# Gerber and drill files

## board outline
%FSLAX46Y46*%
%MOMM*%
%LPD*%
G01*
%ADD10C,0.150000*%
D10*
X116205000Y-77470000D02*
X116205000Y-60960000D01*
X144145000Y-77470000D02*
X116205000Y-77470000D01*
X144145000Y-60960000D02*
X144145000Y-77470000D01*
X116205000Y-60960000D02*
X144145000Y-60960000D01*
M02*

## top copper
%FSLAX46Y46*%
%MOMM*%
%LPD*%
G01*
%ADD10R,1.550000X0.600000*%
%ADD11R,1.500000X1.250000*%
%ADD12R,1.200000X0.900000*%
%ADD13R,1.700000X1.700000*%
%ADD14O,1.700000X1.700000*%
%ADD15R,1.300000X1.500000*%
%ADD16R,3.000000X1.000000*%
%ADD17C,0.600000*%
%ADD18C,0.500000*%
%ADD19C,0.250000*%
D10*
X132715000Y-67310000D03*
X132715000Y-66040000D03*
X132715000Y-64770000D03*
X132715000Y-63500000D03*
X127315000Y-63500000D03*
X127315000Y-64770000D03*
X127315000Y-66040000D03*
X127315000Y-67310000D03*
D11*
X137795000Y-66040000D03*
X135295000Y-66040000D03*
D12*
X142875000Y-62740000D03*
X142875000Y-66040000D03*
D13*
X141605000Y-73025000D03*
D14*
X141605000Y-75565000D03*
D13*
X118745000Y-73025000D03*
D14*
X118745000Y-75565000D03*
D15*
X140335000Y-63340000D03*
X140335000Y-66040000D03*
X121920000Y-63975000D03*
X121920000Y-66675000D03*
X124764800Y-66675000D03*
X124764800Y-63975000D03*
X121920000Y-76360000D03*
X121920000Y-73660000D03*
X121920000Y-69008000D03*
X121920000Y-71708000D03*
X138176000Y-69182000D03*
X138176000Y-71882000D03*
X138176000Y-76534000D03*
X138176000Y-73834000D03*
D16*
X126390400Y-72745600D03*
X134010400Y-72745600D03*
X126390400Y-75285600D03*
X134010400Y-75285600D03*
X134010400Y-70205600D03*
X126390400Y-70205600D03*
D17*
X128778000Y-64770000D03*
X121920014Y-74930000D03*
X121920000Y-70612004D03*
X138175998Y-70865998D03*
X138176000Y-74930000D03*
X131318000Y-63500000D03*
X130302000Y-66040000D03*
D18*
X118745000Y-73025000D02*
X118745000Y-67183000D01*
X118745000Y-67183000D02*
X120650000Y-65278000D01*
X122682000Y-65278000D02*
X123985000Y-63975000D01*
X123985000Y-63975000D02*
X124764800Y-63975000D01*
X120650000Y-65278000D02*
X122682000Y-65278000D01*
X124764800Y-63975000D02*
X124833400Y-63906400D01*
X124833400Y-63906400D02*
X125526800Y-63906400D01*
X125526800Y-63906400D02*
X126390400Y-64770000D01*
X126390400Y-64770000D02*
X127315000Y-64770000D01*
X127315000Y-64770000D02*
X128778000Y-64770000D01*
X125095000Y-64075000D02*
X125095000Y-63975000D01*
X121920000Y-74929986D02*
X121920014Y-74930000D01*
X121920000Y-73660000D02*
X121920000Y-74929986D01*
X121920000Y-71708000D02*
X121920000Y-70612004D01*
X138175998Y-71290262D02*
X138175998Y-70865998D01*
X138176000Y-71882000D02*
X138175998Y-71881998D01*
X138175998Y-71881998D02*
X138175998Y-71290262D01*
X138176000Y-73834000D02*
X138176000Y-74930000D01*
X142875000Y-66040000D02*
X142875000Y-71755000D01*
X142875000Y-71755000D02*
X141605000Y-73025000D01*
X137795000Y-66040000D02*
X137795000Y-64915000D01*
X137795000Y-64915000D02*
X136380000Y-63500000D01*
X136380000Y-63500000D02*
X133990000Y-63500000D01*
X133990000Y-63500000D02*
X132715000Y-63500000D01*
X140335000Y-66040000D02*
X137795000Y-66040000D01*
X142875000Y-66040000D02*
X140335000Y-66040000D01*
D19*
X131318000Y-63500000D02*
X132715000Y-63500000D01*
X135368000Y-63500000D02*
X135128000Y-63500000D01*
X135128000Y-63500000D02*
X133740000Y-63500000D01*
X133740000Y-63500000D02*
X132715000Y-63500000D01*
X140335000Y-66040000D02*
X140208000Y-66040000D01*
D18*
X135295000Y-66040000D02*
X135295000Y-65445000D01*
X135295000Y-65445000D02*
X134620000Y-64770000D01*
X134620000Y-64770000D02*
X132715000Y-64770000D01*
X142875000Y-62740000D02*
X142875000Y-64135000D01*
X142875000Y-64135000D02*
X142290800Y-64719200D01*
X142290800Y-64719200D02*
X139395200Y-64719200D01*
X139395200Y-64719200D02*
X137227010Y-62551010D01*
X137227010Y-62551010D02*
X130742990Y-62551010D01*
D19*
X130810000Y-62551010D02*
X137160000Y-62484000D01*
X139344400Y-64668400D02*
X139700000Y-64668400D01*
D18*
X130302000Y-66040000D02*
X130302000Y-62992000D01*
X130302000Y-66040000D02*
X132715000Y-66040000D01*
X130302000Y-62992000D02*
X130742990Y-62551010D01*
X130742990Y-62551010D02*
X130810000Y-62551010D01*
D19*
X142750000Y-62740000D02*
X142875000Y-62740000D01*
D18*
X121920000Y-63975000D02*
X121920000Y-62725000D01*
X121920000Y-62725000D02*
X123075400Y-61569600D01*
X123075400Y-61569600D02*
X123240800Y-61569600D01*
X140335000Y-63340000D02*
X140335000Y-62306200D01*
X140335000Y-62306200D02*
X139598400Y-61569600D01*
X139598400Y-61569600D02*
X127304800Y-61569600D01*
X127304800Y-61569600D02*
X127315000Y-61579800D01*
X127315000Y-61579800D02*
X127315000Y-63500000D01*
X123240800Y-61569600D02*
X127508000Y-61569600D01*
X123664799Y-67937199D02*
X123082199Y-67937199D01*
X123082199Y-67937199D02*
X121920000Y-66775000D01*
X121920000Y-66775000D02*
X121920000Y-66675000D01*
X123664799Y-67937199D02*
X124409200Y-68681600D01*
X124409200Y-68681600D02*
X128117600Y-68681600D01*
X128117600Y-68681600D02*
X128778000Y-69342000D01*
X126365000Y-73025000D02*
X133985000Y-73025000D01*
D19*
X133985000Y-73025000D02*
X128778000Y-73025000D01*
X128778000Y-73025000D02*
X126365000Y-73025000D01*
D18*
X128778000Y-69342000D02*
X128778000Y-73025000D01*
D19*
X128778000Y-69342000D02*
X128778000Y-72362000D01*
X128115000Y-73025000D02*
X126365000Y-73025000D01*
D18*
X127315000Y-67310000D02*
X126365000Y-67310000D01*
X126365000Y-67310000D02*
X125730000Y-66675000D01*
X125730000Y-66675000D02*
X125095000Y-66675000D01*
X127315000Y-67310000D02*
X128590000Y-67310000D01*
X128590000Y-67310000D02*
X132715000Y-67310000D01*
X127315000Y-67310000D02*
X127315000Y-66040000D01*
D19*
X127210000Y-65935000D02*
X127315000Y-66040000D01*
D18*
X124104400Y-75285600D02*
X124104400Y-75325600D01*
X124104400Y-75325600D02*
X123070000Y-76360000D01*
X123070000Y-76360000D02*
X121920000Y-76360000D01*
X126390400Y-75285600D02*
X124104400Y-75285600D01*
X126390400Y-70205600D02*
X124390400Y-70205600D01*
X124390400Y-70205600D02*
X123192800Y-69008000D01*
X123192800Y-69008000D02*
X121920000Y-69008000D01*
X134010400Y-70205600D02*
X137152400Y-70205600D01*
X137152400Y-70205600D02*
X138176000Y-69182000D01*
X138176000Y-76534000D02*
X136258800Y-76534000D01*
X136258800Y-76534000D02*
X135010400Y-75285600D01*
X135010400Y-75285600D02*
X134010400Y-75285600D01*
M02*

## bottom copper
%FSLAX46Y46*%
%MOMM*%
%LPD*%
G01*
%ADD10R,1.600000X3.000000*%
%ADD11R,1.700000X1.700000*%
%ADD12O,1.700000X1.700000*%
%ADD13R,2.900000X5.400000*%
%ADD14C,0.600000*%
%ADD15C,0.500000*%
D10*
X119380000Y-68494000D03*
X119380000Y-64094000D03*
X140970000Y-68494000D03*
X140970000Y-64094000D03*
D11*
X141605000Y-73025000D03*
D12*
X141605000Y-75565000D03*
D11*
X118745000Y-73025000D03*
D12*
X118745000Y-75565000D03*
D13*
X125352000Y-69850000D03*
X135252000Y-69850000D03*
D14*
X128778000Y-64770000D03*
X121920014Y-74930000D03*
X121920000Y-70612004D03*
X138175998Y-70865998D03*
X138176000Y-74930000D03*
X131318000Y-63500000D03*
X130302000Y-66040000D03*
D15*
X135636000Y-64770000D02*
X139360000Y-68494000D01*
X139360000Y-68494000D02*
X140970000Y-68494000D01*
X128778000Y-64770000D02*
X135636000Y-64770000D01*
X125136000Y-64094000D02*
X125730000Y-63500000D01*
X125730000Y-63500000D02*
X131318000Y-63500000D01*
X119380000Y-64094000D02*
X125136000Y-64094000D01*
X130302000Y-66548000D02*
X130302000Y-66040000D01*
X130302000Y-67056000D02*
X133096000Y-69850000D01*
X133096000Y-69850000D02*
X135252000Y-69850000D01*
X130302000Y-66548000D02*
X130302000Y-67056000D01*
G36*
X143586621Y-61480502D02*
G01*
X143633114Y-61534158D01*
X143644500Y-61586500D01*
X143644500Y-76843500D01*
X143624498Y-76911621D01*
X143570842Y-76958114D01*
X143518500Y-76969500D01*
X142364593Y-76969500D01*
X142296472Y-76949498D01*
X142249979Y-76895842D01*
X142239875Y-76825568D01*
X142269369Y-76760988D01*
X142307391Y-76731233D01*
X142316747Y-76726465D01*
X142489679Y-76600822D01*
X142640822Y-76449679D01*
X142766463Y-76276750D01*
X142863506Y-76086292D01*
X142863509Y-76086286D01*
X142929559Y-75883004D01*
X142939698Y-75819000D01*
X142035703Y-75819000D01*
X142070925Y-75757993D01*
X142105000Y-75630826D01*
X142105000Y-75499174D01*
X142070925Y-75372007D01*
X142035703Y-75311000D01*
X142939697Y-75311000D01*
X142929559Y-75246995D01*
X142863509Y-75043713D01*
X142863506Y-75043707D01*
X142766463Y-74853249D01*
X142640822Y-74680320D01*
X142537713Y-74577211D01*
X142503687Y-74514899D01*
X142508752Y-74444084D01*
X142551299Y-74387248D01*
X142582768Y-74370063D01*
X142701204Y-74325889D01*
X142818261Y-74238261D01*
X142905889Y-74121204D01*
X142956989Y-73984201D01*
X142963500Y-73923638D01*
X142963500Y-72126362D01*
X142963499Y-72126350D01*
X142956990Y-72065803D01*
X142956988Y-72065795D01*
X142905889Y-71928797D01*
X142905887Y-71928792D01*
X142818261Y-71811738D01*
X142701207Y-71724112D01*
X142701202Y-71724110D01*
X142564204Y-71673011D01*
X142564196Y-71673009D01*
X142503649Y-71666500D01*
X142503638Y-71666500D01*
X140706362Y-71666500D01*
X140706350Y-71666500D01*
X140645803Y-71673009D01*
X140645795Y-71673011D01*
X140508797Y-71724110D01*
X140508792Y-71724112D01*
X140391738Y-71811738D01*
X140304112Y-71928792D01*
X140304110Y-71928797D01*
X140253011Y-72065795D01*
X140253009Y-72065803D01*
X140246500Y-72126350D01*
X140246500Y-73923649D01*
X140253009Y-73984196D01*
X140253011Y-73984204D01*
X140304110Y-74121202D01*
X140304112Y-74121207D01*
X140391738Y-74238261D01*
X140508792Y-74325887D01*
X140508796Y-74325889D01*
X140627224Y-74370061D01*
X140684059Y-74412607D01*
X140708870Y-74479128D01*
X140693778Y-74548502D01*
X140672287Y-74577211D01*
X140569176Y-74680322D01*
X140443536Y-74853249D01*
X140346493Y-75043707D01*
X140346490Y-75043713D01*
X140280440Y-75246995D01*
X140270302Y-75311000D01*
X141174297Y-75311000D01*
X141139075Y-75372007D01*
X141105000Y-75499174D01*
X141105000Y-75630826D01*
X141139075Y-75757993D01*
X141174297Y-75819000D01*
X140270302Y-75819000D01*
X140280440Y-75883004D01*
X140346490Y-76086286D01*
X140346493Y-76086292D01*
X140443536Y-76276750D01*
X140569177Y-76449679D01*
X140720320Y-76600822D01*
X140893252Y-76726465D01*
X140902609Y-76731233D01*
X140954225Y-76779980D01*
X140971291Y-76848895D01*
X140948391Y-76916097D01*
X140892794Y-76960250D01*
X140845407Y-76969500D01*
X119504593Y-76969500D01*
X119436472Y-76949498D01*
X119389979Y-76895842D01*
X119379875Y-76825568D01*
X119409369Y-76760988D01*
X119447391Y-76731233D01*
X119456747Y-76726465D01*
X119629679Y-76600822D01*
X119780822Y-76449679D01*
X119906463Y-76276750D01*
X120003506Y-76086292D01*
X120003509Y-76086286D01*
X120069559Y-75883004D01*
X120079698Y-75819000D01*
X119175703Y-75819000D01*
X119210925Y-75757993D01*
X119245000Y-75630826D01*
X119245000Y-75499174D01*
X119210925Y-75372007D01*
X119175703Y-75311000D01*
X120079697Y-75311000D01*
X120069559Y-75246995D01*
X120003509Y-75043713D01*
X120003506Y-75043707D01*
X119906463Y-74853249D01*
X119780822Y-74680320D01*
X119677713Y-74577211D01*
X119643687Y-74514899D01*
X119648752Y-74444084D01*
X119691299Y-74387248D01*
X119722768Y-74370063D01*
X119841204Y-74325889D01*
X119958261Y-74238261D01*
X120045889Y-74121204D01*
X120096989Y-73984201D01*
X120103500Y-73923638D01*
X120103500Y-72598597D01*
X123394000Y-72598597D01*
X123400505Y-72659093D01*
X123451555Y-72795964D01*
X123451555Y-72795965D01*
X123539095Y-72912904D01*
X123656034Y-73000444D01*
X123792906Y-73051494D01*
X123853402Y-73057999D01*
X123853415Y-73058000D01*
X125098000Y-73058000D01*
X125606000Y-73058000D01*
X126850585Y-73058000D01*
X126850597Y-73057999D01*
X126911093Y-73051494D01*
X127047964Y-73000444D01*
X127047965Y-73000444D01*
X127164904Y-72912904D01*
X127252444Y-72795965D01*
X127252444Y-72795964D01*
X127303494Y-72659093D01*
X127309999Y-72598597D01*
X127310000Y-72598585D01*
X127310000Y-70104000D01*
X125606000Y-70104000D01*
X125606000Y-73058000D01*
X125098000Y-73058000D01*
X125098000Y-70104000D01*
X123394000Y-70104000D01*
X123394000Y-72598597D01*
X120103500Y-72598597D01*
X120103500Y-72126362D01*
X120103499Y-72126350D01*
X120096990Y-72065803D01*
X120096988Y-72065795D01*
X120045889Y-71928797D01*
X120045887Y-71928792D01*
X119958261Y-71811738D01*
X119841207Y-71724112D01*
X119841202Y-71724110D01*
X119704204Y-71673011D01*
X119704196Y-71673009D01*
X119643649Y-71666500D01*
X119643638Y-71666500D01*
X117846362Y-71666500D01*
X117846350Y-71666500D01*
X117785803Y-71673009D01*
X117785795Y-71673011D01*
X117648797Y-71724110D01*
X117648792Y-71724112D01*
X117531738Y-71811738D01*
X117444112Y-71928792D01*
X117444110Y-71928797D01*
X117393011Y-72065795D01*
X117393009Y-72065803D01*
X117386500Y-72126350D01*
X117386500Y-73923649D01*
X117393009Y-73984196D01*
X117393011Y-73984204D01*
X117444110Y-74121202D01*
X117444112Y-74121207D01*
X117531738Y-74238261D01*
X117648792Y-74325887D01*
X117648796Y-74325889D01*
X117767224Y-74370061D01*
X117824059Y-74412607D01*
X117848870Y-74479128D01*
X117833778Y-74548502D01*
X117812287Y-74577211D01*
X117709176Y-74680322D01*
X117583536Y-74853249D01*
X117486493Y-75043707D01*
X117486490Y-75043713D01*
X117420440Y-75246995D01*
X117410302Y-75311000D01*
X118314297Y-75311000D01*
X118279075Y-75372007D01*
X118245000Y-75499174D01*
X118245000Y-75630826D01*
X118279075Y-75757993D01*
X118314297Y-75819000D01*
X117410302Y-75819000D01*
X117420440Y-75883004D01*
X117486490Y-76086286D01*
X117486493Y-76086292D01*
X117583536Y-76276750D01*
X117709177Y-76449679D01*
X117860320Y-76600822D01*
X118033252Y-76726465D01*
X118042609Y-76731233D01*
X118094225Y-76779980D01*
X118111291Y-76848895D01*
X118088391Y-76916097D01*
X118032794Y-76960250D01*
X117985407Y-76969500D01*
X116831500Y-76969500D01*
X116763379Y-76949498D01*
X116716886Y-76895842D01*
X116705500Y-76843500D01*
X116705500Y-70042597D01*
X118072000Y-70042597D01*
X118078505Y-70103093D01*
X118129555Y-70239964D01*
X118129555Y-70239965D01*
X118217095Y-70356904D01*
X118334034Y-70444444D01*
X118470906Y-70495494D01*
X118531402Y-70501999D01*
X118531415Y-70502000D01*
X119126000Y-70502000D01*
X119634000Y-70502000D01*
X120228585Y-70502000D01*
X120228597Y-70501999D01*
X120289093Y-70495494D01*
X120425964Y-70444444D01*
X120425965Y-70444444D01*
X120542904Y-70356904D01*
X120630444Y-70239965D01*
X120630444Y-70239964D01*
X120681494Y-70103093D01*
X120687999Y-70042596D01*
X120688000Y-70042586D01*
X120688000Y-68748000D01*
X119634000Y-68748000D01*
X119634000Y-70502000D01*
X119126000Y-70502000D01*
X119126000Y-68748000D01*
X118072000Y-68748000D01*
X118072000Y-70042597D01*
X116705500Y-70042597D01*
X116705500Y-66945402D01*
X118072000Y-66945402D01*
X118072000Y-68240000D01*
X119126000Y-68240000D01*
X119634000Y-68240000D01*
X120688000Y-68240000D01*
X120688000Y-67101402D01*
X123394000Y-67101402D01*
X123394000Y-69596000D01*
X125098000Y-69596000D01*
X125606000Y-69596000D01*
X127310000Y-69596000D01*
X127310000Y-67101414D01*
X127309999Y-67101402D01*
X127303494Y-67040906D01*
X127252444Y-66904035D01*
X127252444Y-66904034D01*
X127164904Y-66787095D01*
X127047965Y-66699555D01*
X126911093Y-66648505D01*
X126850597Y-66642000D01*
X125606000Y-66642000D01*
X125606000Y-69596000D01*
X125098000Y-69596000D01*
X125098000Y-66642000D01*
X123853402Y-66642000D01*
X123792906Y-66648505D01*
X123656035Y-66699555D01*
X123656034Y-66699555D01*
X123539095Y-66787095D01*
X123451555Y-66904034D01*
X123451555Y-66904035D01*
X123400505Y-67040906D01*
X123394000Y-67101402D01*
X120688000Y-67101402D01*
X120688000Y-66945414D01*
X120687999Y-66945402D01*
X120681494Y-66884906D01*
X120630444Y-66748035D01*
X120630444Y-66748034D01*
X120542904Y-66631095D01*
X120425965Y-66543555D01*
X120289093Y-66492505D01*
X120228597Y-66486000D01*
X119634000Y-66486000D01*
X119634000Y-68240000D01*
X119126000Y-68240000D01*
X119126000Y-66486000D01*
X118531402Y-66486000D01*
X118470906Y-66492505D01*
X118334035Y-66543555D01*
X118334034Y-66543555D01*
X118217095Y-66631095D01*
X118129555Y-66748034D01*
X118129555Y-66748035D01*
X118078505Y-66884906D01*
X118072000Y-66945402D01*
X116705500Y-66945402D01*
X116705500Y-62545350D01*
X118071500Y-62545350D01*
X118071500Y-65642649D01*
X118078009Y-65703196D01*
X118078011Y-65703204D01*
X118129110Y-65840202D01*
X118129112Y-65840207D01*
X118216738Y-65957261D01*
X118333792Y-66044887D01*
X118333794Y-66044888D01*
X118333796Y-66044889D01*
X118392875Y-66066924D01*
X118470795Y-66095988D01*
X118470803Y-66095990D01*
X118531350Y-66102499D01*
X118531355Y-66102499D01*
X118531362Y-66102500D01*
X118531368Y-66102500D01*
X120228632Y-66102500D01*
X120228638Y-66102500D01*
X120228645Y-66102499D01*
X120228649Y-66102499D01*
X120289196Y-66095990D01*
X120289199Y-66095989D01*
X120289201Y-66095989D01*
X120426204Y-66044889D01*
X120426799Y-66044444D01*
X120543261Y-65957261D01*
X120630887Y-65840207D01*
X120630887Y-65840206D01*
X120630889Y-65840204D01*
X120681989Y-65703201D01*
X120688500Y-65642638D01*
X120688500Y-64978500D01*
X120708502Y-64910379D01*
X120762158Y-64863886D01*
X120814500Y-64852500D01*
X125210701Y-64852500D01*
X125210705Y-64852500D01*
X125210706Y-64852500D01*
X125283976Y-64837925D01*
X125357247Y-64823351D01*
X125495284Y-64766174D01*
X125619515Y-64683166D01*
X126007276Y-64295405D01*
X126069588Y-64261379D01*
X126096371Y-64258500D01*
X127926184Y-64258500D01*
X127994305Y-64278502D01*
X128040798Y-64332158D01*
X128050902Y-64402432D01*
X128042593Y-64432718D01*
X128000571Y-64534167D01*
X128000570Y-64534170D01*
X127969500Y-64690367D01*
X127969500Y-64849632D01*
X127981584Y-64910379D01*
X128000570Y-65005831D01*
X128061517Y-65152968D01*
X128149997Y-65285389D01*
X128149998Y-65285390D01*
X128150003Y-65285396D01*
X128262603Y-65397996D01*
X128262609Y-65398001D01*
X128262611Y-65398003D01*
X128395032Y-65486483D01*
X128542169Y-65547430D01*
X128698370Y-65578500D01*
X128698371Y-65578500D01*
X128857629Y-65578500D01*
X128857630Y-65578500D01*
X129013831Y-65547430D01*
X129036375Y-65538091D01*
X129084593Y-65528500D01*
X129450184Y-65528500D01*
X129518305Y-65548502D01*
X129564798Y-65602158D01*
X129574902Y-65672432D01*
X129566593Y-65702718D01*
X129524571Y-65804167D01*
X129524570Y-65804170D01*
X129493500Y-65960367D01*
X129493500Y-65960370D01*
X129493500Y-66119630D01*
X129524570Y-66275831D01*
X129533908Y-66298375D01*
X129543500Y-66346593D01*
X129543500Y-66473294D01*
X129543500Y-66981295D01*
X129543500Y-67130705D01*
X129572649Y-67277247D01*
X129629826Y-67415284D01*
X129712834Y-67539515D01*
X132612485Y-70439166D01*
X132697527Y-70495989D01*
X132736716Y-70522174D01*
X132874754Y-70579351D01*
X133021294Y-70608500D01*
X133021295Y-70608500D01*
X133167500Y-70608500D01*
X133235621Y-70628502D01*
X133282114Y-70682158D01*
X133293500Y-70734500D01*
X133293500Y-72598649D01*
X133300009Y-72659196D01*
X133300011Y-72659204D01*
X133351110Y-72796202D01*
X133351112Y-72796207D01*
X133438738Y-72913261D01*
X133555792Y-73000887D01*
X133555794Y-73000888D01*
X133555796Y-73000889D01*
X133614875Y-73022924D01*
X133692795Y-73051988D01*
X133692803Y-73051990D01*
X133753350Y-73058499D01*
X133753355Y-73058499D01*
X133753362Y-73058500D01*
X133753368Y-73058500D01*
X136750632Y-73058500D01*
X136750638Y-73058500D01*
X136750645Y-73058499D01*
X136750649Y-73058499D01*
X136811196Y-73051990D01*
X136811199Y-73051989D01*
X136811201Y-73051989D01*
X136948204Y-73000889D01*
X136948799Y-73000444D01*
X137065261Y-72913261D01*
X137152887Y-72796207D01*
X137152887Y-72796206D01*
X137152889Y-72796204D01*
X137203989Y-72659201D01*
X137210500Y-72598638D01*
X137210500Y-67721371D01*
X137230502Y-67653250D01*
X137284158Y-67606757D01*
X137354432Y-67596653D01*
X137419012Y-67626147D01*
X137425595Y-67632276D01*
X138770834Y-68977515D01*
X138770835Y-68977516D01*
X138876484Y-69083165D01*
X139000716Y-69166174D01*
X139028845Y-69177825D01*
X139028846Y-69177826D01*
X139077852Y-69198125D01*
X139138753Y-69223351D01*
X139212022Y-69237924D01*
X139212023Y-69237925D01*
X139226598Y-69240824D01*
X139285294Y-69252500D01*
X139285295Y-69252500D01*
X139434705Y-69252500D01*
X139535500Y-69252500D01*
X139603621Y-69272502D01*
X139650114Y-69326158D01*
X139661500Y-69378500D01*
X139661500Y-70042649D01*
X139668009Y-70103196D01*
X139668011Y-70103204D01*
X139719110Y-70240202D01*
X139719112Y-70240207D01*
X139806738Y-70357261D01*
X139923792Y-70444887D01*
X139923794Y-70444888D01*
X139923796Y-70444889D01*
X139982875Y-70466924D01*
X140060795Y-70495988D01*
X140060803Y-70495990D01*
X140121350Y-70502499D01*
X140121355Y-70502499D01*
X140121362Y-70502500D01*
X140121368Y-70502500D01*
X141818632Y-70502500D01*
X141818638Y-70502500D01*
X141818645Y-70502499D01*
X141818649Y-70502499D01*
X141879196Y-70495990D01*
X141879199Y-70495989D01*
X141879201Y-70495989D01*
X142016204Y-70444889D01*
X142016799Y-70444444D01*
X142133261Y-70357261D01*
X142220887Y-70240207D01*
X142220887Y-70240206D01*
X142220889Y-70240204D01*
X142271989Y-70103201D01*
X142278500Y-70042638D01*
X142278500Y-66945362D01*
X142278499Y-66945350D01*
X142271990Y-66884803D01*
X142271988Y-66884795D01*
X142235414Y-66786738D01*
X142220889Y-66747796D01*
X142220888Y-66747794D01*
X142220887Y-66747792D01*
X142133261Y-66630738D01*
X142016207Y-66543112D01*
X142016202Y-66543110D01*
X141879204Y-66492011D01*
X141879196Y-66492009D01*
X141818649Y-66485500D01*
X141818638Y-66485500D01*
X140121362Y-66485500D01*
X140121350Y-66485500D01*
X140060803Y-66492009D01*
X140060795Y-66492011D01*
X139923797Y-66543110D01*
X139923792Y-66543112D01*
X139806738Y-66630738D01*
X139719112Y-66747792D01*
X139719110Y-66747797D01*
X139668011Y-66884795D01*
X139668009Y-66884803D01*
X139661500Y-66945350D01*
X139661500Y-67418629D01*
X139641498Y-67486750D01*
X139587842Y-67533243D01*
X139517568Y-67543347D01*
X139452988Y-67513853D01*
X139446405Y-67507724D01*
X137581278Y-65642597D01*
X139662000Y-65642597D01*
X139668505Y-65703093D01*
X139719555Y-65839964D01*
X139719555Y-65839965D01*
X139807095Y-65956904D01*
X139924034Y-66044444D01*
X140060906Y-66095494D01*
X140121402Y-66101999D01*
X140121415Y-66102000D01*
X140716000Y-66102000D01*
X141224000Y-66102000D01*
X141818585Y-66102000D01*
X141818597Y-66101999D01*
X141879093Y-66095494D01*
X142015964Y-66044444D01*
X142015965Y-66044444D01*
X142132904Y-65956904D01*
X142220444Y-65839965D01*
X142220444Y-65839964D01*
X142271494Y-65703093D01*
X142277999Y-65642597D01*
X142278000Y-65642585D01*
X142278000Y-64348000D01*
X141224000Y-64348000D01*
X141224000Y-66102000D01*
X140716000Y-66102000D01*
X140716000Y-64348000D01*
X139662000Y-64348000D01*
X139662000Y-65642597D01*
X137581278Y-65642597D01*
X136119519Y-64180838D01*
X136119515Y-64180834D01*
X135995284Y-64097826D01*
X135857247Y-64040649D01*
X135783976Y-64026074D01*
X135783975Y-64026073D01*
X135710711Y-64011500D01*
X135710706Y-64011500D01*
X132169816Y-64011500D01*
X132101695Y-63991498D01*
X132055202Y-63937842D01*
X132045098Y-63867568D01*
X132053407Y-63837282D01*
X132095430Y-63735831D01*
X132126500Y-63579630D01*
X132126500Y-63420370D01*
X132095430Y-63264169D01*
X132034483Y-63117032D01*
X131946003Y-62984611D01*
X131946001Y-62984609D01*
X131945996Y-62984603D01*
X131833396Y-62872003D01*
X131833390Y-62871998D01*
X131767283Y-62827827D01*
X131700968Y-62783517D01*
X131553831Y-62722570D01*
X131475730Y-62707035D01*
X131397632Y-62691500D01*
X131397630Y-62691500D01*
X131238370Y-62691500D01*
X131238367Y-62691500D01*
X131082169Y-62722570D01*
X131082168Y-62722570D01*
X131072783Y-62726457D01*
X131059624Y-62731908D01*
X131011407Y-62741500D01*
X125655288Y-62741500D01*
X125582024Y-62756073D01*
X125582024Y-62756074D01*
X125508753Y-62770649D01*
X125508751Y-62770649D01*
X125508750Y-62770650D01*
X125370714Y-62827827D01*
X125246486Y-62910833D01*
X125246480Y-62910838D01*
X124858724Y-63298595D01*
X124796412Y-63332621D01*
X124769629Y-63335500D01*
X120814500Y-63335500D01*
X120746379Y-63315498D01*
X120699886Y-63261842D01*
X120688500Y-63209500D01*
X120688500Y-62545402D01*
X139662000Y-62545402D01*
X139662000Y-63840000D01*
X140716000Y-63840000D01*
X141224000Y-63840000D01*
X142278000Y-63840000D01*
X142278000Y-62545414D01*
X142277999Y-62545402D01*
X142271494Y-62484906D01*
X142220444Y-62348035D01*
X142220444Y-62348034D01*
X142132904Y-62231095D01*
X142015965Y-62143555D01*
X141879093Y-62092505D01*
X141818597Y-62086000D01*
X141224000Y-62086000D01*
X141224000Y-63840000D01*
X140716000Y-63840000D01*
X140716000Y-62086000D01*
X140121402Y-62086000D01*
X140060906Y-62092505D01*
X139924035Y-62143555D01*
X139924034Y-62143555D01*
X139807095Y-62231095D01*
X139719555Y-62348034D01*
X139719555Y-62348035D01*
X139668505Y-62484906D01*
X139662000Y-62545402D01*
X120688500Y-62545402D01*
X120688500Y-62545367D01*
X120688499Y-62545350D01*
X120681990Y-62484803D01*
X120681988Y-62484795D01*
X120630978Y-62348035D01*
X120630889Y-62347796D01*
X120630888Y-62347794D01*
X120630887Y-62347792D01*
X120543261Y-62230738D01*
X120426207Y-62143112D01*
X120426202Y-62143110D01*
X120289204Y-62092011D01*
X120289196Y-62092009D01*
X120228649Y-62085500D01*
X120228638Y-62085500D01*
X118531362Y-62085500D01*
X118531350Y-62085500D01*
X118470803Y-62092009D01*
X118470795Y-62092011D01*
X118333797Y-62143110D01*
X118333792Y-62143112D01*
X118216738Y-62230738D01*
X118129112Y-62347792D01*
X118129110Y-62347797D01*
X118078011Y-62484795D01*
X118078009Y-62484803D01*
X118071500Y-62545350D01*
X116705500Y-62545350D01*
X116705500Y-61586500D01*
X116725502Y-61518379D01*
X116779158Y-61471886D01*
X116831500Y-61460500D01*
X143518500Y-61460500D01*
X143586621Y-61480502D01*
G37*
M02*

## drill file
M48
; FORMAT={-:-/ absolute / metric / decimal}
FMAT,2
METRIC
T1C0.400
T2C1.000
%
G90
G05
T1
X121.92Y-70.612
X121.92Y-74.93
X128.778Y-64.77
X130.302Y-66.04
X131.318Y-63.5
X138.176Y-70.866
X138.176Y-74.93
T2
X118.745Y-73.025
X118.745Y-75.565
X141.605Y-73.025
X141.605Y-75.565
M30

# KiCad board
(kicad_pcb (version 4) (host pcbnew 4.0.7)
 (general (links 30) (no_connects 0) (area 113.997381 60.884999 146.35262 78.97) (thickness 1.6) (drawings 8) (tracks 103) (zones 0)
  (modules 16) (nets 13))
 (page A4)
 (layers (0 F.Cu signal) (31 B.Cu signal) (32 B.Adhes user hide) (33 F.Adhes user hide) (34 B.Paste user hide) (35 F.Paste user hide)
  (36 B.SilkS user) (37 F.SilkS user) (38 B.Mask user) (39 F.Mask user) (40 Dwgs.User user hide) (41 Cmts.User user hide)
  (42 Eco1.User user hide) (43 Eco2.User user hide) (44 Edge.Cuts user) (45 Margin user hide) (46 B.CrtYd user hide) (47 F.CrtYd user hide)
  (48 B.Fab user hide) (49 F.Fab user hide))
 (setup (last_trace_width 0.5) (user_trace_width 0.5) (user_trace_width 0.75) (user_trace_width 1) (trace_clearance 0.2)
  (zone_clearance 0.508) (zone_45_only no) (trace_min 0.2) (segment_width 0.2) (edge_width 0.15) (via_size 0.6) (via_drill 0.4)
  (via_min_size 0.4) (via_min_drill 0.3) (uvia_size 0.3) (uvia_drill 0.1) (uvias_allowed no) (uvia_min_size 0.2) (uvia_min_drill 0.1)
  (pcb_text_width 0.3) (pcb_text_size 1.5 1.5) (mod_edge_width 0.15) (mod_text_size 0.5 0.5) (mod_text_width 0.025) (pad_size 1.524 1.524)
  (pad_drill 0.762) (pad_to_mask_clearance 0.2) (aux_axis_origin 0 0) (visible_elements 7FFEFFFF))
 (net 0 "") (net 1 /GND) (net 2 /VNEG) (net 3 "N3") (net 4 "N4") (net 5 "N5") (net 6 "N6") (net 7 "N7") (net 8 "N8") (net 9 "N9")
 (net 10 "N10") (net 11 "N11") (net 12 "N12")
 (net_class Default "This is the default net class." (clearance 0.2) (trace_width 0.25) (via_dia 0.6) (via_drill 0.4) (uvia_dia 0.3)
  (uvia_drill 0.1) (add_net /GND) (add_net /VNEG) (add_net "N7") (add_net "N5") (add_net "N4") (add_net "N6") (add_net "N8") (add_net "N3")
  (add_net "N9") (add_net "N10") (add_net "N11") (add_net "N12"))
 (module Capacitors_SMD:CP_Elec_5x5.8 (layer B.Cu) (at 119.38 66.294 90)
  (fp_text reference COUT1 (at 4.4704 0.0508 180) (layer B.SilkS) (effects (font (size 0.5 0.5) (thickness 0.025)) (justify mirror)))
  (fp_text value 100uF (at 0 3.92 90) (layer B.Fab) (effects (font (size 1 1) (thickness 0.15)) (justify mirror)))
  (pad 1 smd rect (at -2.2 0 270) (size 3 1.6) (layers B.Cu B.Paste B.Mask) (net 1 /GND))
  (pad 2 smd rect (at 2.2 0 270) (size 3 1.6) (layers B.Cu B.Paste B.Mask) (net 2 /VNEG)))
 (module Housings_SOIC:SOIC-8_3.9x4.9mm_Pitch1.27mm (layer F.Cu) (at 130.015 65.405 180)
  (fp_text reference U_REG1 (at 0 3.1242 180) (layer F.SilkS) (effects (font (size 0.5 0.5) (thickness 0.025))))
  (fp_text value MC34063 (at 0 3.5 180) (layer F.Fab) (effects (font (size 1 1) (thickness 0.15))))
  (pad 1 smd rect (at -2.7 -1.905 180) (size 1.55 0.6) (layers F.Cu F.Paste F.Mask) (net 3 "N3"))
  (pad 2 smd rect (at -2.7 -0.635 180) (size 1.55 0.6) (layers F.Cu F.Paste F.Mask) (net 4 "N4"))
  (pad 3 smd rect (at -2.7 0.635 180) (size 1.55 0.6) (layers F.Cu F.Paste F.Mask) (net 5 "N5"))
  (pad 4 smd rect (at -2.7 1.905 180) (size 1.55 0.6) (layers F.Cu F.Paste F.Mask) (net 2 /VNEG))
  (pad 5 smd rect (at 2.7 1.905 180) (size 1.55 0.6) (layers F.Cu F.Paste F.Mask) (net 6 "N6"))
  (pad 6 smd rect (at 2.7 0.635 180) (size 1.55 0.6) (layers F.Cu F.Paste F.Mask) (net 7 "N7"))
  (pad 7 smd rect (at 2.7 -0.635 180) (size 1.55 0.6) (layers F.Cu F.Paste F.Mask) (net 3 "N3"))
  (pad 8 smd rect (at 2.7 -1.905 180) (size 1.55 0.6) (layers F.Cu F.Paste F.Mask) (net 3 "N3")))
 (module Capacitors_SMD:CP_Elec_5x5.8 (layer B.Cu) (at 140.97 66.294 90)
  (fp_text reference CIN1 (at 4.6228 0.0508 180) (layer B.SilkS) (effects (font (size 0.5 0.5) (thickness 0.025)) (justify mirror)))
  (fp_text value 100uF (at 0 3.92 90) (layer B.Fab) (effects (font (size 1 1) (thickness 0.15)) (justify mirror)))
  (pad 1 smd rect (at -2.2 0 270) (size 3 1.6) (layers B.Cu B.Paste B.Mask) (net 7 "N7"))
  (pad 2 smd rect (at 2.2 0 270) (size 3 1.6) (layers B.Cu B.Paste B.Mask) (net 1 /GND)))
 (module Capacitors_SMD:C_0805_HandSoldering (layer F.Cu) (at 136.545 66.04 180)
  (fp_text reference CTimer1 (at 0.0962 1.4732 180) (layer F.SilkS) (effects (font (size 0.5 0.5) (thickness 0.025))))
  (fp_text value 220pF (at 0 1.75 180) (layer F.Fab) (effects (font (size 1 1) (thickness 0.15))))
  (pad 1 smd rect (at -1.25 0 180) (size 1.5 1.25) (layers F.Cu F.Paste F.Mask) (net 2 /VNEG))
  (pad 2 smd rect (at 1.25 0 180) (size 1.5 1.25) (layers F.Cu F.Paste F.Mask) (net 5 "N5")))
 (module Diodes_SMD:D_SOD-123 (layer F.Cu) (at 142.875 64.39 270)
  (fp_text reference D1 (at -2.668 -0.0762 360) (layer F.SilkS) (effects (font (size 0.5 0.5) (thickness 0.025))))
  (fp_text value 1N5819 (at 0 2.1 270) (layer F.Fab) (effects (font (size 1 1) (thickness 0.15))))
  (pad 1 smd rect (at -1.65 0 270) (size 0.9 1.2) (layers F.Cu F.Paste F.Mask) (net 4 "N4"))
  (pad 2 smd rect (at 1.65 0 270) (size 0.9 1.2) (layers F.Cu F.Paste F.Mask) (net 2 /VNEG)))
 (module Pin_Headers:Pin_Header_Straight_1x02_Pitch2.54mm (layer F.Cu) (at 141.605 73.025)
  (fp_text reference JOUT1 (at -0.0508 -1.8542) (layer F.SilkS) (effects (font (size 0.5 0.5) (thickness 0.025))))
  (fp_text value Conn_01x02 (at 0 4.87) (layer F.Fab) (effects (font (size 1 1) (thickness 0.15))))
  (pad 1 thru_hole rect (at 0 0) (size 1.7 1.7) (drill 1) (layers *.Cu *.Mask) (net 2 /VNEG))
  (pad 2 thru_hole oval (at 0 2.54) (size 1.7 1.7) (drill 1) (layers *.Cu *.Mask) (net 1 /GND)))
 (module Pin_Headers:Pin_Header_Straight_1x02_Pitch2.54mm (layer F.Cu) (at 118.745 73.025)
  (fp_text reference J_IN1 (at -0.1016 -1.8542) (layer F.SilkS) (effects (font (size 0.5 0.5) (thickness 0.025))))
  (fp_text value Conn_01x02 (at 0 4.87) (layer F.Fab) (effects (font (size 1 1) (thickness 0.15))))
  (pad 1 thru_hole rect (at 0 0) (size 1.7 1.7) (drill 1) (layers *.Cu *.Mask) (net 7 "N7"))
  (pad 2 thru_hole oval (at 0 2.54) (size 1.7 1.7) (drill 1) (layers *.Cu *.Mask) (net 1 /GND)))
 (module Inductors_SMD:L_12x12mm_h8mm (layer B.Cu) (at 130.302 69.85)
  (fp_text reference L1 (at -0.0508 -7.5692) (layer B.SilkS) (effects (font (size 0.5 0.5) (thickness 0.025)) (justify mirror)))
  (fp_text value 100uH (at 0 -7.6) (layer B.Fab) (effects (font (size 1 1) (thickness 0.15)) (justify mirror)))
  (pad 1 smd rect (at -4.95 0) (size 2.9 5.4) (layers B.Cu B.Paste B.Mask) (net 1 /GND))
  (pad 2 smd rect (at 4.95 0) (size 2.9 5.4) (layers B.Cu B.Paste B.Mask) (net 4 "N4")))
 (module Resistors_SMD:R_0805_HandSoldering (layer F.Cu) (at 140.335 64.69 270)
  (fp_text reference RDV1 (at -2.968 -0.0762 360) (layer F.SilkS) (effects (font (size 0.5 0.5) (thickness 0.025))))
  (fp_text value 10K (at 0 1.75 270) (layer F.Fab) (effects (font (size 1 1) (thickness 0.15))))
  (pad 1 smd rect (at -1.35 0 270) (size 1.5 1.3) (layers F.Cu F.Paste F.Mask) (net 6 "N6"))
  (pad 2 smd rect (at 1.35 0 270) (size 1.5 1.3) (layers F.Cu F.Paste F.Mask) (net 2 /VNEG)))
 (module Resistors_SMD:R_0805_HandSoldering (layer F.Cu) (at 121.92 65.325 270)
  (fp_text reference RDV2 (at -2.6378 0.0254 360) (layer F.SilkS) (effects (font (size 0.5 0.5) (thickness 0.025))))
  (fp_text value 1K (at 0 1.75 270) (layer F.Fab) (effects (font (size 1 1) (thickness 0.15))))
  (pad 1 smd rect (at -1.35 0 270) (size 1.5 1.3) (layers F.Cu F.Paste F.Mask) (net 6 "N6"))
  (pad 2 smd rect (at 1.35 0 270) (size 1.5 1.3) (layers F.Cu F.Paste F.Mask) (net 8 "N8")))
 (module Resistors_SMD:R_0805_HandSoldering (layer F.Cu) (at 124.7648 65.325 90)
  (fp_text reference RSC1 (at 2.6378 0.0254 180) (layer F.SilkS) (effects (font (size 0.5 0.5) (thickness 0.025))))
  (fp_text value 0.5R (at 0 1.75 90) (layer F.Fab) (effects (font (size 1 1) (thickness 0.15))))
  (pad 1 smd rect (at -1.35 0 90) (size 1.5 1.3) (layers F.Cu F.Paste F.Mask) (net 3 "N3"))
  (pad 2 smd rect (at 1.35 0 90) (size 1.5 1.3) (layers F.Cu F.Paste F.Mask) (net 7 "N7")))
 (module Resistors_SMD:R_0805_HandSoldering (layer F.Cu) (at 121.92 75.01 90)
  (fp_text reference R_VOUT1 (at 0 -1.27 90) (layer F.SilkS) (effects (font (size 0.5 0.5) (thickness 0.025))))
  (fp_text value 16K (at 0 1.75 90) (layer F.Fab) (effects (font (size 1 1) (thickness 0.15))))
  (pad 1 smd rect (at -1.35 0 90) (size 1.5 1.3) (layers F.Cu F.Paste F.Mask) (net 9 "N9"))
  (pad 2 smd rect (at 1.35 0 90) (size 1.5 1.3) (layers F.Cu F.Paste F.Mask) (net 1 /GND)))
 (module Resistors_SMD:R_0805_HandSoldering (layer F.Cu) (at 121.92 70.358 270)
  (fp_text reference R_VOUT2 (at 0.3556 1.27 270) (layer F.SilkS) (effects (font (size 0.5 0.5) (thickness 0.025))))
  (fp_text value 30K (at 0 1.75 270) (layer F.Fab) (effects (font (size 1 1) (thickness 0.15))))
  (pad 1 smd rect (at -1.35 0 270) (size 1.5 1.3) (layers F.Cu F.Paste F.Mask) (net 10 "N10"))
  (pad 2 smd rect (at 1.35 0 270) (size 1.5 1.3) (layers F.Cu F.Paste F.Mask) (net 1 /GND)))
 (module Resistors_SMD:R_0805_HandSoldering (layer F.Cu) (at 138.176 70.532 270)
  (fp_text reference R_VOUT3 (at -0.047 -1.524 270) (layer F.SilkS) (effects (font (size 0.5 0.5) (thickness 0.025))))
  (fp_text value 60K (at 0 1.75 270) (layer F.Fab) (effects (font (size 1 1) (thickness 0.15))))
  (pad 1 smd rect (at -1.35 0 270) (size 1.5 1.3) (layers F.Cu F.Paste F.Mask) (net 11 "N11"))
  (pad 2 smd rect (at 1.35 0 270) (size 1.5 1.3) (layers F.Cu F.Paste F.Mask) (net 1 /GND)))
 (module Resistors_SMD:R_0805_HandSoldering (layer F.Cu) (at 138.176 75.184 90)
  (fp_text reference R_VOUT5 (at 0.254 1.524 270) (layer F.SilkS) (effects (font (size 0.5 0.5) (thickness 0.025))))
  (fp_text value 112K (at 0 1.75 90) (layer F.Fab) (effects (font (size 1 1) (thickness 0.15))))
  (pad 1 smd rect (at -1.35 0 90) (size 1.5 1.3) (layers F.Cu F.Paste F.Mask) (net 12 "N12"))
  (pad 2 smd rect (at 1.35 0 90) (size 1.5 1.3) (layers F.Cu F.Paste F.Mask) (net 1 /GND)))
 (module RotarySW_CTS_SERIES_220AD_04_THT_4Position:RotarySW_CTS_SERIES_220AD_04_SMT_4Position (layer F.Cu) (at 130.2004 72.7456)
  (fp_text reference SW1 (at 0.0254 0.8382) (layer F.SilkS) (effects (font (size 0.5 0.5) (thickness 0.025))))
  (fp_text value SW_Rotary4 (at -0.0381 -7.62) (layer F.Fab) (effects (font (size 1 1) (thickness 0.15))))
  (pad 4 smd rect (at -3.81 0) (size 3 1) (layers F.Cu F.Paste F.Mask) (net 8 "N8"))
  (pad 4 smd rect (at 3.81 0) (size 3 1) (layers F.Cu F.Paste F.Mask) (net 8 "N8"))
  (pad 0 smd rect (at -3.81 2.54 180) (size 3 1) (layers F.Cu F.Paste F.Mask) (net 9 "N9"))
  (pad 3 smd rect (at 3.81 2.54) (size 3 1) (layers F.Cu F.Paste F.Mask) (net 12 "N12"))
  (pad 2 smd rect (at 3.81 -2.54) (size 3 1) (layers F.Cu F.Paste F.Mask) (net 11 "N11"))
  (pad 1 smd rect (at -3.81 -2.54) (size 3 1) (layers F.Cu F.Paste F.Mask) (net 10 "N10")))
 (gr_line (start 116.205 77.47) (end 116.205 60.96) (layer Edge.Cuts) (width 0.15))
 (gr_line (start 144.145 77.47) (end 116.205 77.47) (layer Edge.Cuts) (width 0.15))
 (gr_line (start 144.145 60.96) (end 144.145 77.47) (layer Edge.Cuts) (width 0.15))
 (gr_line (start 116.205 60.96) (end 144.145 60.96) (layer Edge.Cuts) (width 0.15))
 (segment (start 118.745 73.025) (end 118.745 67.183) (width 0.5) (layer F.Cu) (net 7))
 (segment (start 118.745 67.183) (end 120.65 65.278) (width 0.5) (layer F.Cu) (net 7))
 (segment (start 122.682 65.278) (end 123.985 63.975) (width 0.5) (layer F.Cu) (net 7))
 (segment (start 123.985 63.975) (end 124.7648 63.975) (width 0.5) (layer F.Cu) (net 7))
 (segment (start 120.65 65.278) (end 122.682 65.278) (width 0.5) (layer F.Cu) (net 7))
 (segment (start 124.7648 63.975) (end 124.8334 63.9064) (width 0.5) (layer F.Cu) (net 7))
 (segment (start 124.8334 63.9064) (end 125.5268 63.9064) (width 0.5) (layer F.Cu) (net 7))
 (segment (start 125.5268 63.9064) (end 126.3904 64.77) (width 0.5) (layer F.Cu) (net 7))
 (segment (start 126.3904 64.77) (end 127.315 64.77) (width 0.5) (layer F.Cu) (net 7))
 (segment (start 135.636 64.77) (end 139.36 68.494) (width 0.5) (layer B.Cu) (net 7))
 (segment (start 139.36 68.494) (end 140.97 68.494) (width 0.5) (layer B.Cu) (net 7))
 (segment (start 128.778 64.77) (end 135.636 64.77) (width 0.5) (layer B.Cu) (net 7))
 (segment (start 127.315 64.77) (end 128.778 64.77) (width 0.5) (layer F.Cu) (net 7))
 (segment (start 125.095 64.075) (end 125.095 63.975) (width 0.5) (layer F.Cu) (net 7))
 (via (at 128.778 64.77) (size 0.6) (drill 0.4) (layers F.Cu B.Cu) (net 7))
 (segment (start 121.92 74.929986) (end 121.920014 74.93) (width 0.5) (layer F.Cu) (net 1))
 (segment (start 121.92 73.66) (end 121.92 74.929986) (width 0.5) (layer F.Cu) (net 1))
 (via (at 121.920014 74.93) (size 0.6) (drill 0.4) (layers F.Cu B.Cu) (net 1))
 (segment (start 121.92 71.708) (end 121.92 70.612004) (width 0.5) (layer F.Cu) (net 1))
 (via (at 121.92 70.612004) (size 0.6) (drill 0.4) (layers F.Cu B.Cu) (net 1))
 (segment (start 138.175998 71.290262) (end 138.175998 70.865998) (width 0.5) (layer F.Cu) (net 1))
 (segment (start 138.176 71.882) (end 138.175998 71.881998) (width 0.5) (layer F.Cu) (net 1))
 (segment (start 138.175998 71.881998) (end 138.175998 71.290262) (width 0.5) (layer F.Cu) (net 1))
 (via (at 138.175998 70.865998) (size 0.6) (drill 0.4) (layers F.Cu B.Cu) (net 1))
 (via (at 138.176 74.93) (size 0.6) (drill 0.4) (layers F.Cu B.Cu) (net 1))
 (segment (start 138.176 73.834) (end 138.176 74.93) (width 0.5) (layer F.Cu) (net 1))
 (segment (start 142.875 66.04) (end 142.875 71.755) (width 0.5) (layer F.Cu) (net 2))
 (segment (start 142.875 71.755) (end 141.605 73.025) (width 0.5) (layer F.Cu) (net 2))
 (segment (start 137.795 66.04) (end 137.795 64.915) (width 0.5) (layer F.Cu) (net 2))
 (segment (start 137.795 64.915) (end 136.38 63.5) (width 0.5) (layer F.Cu) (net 2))
 (segment (start 136.38 63.5) (end 133.99 63.5) (width 0.5) (layer F.Cu) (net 2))
 (segment (start 133.99 63.5) (end 132.715 63.5) (width 0.5) (layer F.Cu) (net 2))
 (segment (start 140.335 66.04) (end 137.795 66.04) (width 0.5) (layer F.Cu) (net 2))
 (segment (start 142.875 66.04) (end 140.335 66.04) (width 0.5) (layer F.Cu) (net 2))
 (segment (start 125.136 64.094) (end 125.73 63.5) (width 0.5) (layer B.Cu) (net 2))
 (segment (start 125.73 63.5) (end 131.318 63.5) (width 0.5) (layer B.Cu) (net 2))
 (segment (start 119.38 64.094) (end 125.136 64.094) (width 0.5) (layer B.Cu) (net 2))
 (segment (start 131.318 63.5) (end 132.715 63.5) (width 0.25) (layer F.Cu) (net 2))
 (via (at 131.318 63.5) (size 0.6) (drill 0.4) (layers F.Cu B.Cu) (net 2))
 (segment (start 135.368 63.5) (end 135.128 63.5) (width 0.25) (layer F.Cu) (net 2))
 (segment (start 135.128 63.5) (end 133.74 63.5) (width 0.25) (layer F.Cu) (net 2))
 (segment (start 133.74 63.5) (end 132.715 63.5) (width 0.25) (layer F.Cu) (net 2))
 (segment (start 140.335 66.04) (end 140.208 66.04) (width 0.25) (layer F.Cu) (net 2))
 (segment (start 135.295 66.04) (end 135.295 65.445) (width 0.5) (layer F.Cu) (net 5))
 (segment (start 135.295 65.445) (end 134.62 64.77) (width 0.5) (layer F.Cu) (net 5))
 (segment (start 134.62 64.77) (end 132.715 64.77) (width 0.5) (layer F.Cu) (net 5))
 (segment (start 142.875 62.74) (end 142.875 64.135) (width 0.5) (layer F.Cu) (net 4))
 (segment (start 142.875 64.135) (end 142.2908 64.7192) (width 0.5) (layer F.Cu) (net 4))
 (segment (start 142.2908 64.7192) (end 139.3952 64.7192) (width 0.5) (layer F.Cu) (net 4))
 (segment (start 139.3952 64.7192) (end 137.22701 62.55101) (width 0.5) (layer F.Cu) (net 4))
 (segment (start 137.22701 62.55101) (end 130.74299 62.55101) (width 0.5) (layer F.Cu) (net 4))
 (segment (start 130.81 62.55101) (end 137.16 62.484) (width 0.25) (layer F.Cu) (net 4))
 (segment (start 139.3444 64.6684) (end 139.7 64.6684) (width 0.25) (layer F.Cu) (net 4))
 (segment (start 130.302 66.548) (end 130.302 66.04) (width 0.5) (layer B.Cu) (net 4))
 (segment (start 130.302 66.04) (end 130.302 62.992) (width 0.5) (layer F.Cu) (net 4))
 (segment (start 130.302 66.04) (end 132.715 66.04) (width 0.5) (layer F.Cu) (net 4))
 (segment (start 130.302 62.992) (end 130.74299 62.55101) (width 0.5) (layer F.Cu) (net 4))
 (segment (start 130.74299 62.55101) (end 130.81 62.55101) (width 0.5) (layer F.Cu) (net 4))
 (segment (start 130.302 67.056) (end 133.096 69.85) (width 0.5) (layer B.Cu) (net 4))
 (segment (start 133.096 69.85) (end 135.252 69.85) (width 0.5) (layer B.Cu) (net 4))
 (segment (start 130.302 66.548) (end 130.302 67.056) (width 0.5) (layer B.Cu) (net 4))
 (via (at 130.302 66.04) (size 0.6) (drill 0.4) (layers F.Cu B.Cu) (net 4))
 (segment (start 142.75 62.74) (end 142.875 62.74) (width 0.25) (layer F.Cu) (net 4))
 (segment (start 121.92 63.975) (end 121.92 62.725) (width 0.5) (layer F.Cu) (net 6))
 (segment (start 121.92 62.725) (end 123.0754 61.5696) (width 0.5) (layer F.Cu) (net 6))
 (segment (start 123.0754 61.5696) (end 123.2408 61.5696) (width 0.5) (layer F.Cu) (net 6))
 (segment (start 140.335 63.34) (end 140.335 62.3062) (width 0.5) (layer F.Cu) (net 6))
 (segment (start 140.335 62.3062) (end 139.5984 61.5696) (width 0.5) (layer F.Cu) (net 6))
 (segment (start 139.5984 61.5696) (end 127.3048 61.5696) (width 0.5) (layer F.Cu) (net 6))
 (segment (start 127.3048 61.5696) (end 127.315 61.5798) (width 0.5) (layer F.Cu) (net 6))
 (segment (start 127.315 61.5798) (end 127.315 63.5) (width 0.5) (layer F.Cu) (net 6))
 (segment (start 123.2408 61.5696) (end 127.508 61.5696) (width 0.5) (layer F.Cu) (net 6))
 (segment (start 123.664799 67.937199) (end 123.082199 67.937199) (width 0.5) (layer F.Cu) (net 8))
 (segment (start 123.082199 67.937199) (end 121.92 66.775) (width 0.5) (layer F.Cu) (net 8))
 (segment (start 121.92 66.775) (end 121.92 66.675) (width 0.5) (layer F.Cu) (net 8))
 (segment (start 123.664799 67.937199) (end 124.4092 68.6816) (width 0.5) (layer F.Cu) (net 8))
 (segment (start 124.4092 68.6816) (end 128.1176 68.6816) (width 0.5) (layer F.Cu) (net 8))
 (segment (start 128.1176 68.6816) (end 128.778 69.342) (width 0.5) (layer F.Cu) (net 8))
 (segment (start 126.365 73.025) (end 133.985 73.025) (width 0.5) (layer F.Cu) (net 8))
 (segment (start 133.985 73.025) (end 128.778 73.025) (width 0.25) (layer F.Cu) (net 8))
 (segment (start 128.778 73.025) (end 126.365 73.025) (width 0.25) (layer F.Cu) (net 8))
 (segment (start 128.778 69.342) (end 128.778 73.025) (width 0.5) (layer F.Cu) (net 8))
 (segment (start 128.778 69.342) (end 128.778 72.362) (width 0.25) (layer F.Cu) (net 8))
 (segment (start 128.115 73.025) (end 126.365 73.025) (width 0.25) (layer F.Cu) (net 8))
 (segment (start 127.315 67.31) (end 126.365 67.31) (width 0.5) (layer F.Cu) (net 3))
 (segment (start 126.365 67.31) (end 125.73 66.675) (width 0.5) (layer F.Cu) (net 3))
 (segment (start 125.73 66.675) (end 125.095 66.675) (width 0.5) (layer F.Cu) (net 3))
 (segment (start 127.315 67.31) (end 128.59 67.31) (width 0.5) (layer F.Cu) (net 3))
 (segment (start 128.59 67.31) (end 132.715 67.31) (width 0.5) (layer F.Cu) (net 3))
 (segment (start 127.315 67.31) (end 127.315 66.04) (width 0.5) (layer F.Cu) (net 3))
 (segment (start 127.21 65.935) (end 127.315 66.04) (width 0.25) (layer F.Cu) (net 3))
 (segment (start 124.1044 75.2856) (end 124.1044 75.3256) (width 0.5) (layer F.Cu) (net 9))
 (segment (start 124.1044 75.3256) (end 123.07 76.36) (width 0.5) (layer F.Cu) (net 9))
 (segment (start 123.07 76.36) (end 121.92 76.36) (width 0.5) (layer F.Cu) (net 9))
 (segment (start 126.3904 75.2856) (end 124.1044 75.2856) (width 0.5) (layer F.Cu) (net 9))
 (segment (start 126.3904 70.2056) (end 124.3904 70.2056) (width 0.5) (layer F.Cu) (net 10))
 (segment (start 124.3904 70.2056) (end 123.1928 69.008) (width 0.5) (layer F.Cu) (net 10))
 (segment (start 123.1928 69.008) (end 121.92 69.008) (width 0.5) (layer F.Cu) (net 10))
 (segment (start 134.0104 70.2056) (end 137.1524 70.2056) (width 0.5) (layer F.Cu) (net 11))
 (segment (start 137.1524 70.2056) (end 138.176 69.182) (width 0.5) (layer F.Cu) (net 11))
 (segment (start 138.176 76.534) (end 136.2588 76.534) (width 0.5) (layer F.Cu) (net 12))
 (segment (start 136.2588 76.534) (end 135.0104 75.2856) (width 0.5) (layer F.Cu) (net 12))
 (segment (start 135.0104 75.2856) (end 134.0104 75.2856) (width 0.5) (layer F.Cu) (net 12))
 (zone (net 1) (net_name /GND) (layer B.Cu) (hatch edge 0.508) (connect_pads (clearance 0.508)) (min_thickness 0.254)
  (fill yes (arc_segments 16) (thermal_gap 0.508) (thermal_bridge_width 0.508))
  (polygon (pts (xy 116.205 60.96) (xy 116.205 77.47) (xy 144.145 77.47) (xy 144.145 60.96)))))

